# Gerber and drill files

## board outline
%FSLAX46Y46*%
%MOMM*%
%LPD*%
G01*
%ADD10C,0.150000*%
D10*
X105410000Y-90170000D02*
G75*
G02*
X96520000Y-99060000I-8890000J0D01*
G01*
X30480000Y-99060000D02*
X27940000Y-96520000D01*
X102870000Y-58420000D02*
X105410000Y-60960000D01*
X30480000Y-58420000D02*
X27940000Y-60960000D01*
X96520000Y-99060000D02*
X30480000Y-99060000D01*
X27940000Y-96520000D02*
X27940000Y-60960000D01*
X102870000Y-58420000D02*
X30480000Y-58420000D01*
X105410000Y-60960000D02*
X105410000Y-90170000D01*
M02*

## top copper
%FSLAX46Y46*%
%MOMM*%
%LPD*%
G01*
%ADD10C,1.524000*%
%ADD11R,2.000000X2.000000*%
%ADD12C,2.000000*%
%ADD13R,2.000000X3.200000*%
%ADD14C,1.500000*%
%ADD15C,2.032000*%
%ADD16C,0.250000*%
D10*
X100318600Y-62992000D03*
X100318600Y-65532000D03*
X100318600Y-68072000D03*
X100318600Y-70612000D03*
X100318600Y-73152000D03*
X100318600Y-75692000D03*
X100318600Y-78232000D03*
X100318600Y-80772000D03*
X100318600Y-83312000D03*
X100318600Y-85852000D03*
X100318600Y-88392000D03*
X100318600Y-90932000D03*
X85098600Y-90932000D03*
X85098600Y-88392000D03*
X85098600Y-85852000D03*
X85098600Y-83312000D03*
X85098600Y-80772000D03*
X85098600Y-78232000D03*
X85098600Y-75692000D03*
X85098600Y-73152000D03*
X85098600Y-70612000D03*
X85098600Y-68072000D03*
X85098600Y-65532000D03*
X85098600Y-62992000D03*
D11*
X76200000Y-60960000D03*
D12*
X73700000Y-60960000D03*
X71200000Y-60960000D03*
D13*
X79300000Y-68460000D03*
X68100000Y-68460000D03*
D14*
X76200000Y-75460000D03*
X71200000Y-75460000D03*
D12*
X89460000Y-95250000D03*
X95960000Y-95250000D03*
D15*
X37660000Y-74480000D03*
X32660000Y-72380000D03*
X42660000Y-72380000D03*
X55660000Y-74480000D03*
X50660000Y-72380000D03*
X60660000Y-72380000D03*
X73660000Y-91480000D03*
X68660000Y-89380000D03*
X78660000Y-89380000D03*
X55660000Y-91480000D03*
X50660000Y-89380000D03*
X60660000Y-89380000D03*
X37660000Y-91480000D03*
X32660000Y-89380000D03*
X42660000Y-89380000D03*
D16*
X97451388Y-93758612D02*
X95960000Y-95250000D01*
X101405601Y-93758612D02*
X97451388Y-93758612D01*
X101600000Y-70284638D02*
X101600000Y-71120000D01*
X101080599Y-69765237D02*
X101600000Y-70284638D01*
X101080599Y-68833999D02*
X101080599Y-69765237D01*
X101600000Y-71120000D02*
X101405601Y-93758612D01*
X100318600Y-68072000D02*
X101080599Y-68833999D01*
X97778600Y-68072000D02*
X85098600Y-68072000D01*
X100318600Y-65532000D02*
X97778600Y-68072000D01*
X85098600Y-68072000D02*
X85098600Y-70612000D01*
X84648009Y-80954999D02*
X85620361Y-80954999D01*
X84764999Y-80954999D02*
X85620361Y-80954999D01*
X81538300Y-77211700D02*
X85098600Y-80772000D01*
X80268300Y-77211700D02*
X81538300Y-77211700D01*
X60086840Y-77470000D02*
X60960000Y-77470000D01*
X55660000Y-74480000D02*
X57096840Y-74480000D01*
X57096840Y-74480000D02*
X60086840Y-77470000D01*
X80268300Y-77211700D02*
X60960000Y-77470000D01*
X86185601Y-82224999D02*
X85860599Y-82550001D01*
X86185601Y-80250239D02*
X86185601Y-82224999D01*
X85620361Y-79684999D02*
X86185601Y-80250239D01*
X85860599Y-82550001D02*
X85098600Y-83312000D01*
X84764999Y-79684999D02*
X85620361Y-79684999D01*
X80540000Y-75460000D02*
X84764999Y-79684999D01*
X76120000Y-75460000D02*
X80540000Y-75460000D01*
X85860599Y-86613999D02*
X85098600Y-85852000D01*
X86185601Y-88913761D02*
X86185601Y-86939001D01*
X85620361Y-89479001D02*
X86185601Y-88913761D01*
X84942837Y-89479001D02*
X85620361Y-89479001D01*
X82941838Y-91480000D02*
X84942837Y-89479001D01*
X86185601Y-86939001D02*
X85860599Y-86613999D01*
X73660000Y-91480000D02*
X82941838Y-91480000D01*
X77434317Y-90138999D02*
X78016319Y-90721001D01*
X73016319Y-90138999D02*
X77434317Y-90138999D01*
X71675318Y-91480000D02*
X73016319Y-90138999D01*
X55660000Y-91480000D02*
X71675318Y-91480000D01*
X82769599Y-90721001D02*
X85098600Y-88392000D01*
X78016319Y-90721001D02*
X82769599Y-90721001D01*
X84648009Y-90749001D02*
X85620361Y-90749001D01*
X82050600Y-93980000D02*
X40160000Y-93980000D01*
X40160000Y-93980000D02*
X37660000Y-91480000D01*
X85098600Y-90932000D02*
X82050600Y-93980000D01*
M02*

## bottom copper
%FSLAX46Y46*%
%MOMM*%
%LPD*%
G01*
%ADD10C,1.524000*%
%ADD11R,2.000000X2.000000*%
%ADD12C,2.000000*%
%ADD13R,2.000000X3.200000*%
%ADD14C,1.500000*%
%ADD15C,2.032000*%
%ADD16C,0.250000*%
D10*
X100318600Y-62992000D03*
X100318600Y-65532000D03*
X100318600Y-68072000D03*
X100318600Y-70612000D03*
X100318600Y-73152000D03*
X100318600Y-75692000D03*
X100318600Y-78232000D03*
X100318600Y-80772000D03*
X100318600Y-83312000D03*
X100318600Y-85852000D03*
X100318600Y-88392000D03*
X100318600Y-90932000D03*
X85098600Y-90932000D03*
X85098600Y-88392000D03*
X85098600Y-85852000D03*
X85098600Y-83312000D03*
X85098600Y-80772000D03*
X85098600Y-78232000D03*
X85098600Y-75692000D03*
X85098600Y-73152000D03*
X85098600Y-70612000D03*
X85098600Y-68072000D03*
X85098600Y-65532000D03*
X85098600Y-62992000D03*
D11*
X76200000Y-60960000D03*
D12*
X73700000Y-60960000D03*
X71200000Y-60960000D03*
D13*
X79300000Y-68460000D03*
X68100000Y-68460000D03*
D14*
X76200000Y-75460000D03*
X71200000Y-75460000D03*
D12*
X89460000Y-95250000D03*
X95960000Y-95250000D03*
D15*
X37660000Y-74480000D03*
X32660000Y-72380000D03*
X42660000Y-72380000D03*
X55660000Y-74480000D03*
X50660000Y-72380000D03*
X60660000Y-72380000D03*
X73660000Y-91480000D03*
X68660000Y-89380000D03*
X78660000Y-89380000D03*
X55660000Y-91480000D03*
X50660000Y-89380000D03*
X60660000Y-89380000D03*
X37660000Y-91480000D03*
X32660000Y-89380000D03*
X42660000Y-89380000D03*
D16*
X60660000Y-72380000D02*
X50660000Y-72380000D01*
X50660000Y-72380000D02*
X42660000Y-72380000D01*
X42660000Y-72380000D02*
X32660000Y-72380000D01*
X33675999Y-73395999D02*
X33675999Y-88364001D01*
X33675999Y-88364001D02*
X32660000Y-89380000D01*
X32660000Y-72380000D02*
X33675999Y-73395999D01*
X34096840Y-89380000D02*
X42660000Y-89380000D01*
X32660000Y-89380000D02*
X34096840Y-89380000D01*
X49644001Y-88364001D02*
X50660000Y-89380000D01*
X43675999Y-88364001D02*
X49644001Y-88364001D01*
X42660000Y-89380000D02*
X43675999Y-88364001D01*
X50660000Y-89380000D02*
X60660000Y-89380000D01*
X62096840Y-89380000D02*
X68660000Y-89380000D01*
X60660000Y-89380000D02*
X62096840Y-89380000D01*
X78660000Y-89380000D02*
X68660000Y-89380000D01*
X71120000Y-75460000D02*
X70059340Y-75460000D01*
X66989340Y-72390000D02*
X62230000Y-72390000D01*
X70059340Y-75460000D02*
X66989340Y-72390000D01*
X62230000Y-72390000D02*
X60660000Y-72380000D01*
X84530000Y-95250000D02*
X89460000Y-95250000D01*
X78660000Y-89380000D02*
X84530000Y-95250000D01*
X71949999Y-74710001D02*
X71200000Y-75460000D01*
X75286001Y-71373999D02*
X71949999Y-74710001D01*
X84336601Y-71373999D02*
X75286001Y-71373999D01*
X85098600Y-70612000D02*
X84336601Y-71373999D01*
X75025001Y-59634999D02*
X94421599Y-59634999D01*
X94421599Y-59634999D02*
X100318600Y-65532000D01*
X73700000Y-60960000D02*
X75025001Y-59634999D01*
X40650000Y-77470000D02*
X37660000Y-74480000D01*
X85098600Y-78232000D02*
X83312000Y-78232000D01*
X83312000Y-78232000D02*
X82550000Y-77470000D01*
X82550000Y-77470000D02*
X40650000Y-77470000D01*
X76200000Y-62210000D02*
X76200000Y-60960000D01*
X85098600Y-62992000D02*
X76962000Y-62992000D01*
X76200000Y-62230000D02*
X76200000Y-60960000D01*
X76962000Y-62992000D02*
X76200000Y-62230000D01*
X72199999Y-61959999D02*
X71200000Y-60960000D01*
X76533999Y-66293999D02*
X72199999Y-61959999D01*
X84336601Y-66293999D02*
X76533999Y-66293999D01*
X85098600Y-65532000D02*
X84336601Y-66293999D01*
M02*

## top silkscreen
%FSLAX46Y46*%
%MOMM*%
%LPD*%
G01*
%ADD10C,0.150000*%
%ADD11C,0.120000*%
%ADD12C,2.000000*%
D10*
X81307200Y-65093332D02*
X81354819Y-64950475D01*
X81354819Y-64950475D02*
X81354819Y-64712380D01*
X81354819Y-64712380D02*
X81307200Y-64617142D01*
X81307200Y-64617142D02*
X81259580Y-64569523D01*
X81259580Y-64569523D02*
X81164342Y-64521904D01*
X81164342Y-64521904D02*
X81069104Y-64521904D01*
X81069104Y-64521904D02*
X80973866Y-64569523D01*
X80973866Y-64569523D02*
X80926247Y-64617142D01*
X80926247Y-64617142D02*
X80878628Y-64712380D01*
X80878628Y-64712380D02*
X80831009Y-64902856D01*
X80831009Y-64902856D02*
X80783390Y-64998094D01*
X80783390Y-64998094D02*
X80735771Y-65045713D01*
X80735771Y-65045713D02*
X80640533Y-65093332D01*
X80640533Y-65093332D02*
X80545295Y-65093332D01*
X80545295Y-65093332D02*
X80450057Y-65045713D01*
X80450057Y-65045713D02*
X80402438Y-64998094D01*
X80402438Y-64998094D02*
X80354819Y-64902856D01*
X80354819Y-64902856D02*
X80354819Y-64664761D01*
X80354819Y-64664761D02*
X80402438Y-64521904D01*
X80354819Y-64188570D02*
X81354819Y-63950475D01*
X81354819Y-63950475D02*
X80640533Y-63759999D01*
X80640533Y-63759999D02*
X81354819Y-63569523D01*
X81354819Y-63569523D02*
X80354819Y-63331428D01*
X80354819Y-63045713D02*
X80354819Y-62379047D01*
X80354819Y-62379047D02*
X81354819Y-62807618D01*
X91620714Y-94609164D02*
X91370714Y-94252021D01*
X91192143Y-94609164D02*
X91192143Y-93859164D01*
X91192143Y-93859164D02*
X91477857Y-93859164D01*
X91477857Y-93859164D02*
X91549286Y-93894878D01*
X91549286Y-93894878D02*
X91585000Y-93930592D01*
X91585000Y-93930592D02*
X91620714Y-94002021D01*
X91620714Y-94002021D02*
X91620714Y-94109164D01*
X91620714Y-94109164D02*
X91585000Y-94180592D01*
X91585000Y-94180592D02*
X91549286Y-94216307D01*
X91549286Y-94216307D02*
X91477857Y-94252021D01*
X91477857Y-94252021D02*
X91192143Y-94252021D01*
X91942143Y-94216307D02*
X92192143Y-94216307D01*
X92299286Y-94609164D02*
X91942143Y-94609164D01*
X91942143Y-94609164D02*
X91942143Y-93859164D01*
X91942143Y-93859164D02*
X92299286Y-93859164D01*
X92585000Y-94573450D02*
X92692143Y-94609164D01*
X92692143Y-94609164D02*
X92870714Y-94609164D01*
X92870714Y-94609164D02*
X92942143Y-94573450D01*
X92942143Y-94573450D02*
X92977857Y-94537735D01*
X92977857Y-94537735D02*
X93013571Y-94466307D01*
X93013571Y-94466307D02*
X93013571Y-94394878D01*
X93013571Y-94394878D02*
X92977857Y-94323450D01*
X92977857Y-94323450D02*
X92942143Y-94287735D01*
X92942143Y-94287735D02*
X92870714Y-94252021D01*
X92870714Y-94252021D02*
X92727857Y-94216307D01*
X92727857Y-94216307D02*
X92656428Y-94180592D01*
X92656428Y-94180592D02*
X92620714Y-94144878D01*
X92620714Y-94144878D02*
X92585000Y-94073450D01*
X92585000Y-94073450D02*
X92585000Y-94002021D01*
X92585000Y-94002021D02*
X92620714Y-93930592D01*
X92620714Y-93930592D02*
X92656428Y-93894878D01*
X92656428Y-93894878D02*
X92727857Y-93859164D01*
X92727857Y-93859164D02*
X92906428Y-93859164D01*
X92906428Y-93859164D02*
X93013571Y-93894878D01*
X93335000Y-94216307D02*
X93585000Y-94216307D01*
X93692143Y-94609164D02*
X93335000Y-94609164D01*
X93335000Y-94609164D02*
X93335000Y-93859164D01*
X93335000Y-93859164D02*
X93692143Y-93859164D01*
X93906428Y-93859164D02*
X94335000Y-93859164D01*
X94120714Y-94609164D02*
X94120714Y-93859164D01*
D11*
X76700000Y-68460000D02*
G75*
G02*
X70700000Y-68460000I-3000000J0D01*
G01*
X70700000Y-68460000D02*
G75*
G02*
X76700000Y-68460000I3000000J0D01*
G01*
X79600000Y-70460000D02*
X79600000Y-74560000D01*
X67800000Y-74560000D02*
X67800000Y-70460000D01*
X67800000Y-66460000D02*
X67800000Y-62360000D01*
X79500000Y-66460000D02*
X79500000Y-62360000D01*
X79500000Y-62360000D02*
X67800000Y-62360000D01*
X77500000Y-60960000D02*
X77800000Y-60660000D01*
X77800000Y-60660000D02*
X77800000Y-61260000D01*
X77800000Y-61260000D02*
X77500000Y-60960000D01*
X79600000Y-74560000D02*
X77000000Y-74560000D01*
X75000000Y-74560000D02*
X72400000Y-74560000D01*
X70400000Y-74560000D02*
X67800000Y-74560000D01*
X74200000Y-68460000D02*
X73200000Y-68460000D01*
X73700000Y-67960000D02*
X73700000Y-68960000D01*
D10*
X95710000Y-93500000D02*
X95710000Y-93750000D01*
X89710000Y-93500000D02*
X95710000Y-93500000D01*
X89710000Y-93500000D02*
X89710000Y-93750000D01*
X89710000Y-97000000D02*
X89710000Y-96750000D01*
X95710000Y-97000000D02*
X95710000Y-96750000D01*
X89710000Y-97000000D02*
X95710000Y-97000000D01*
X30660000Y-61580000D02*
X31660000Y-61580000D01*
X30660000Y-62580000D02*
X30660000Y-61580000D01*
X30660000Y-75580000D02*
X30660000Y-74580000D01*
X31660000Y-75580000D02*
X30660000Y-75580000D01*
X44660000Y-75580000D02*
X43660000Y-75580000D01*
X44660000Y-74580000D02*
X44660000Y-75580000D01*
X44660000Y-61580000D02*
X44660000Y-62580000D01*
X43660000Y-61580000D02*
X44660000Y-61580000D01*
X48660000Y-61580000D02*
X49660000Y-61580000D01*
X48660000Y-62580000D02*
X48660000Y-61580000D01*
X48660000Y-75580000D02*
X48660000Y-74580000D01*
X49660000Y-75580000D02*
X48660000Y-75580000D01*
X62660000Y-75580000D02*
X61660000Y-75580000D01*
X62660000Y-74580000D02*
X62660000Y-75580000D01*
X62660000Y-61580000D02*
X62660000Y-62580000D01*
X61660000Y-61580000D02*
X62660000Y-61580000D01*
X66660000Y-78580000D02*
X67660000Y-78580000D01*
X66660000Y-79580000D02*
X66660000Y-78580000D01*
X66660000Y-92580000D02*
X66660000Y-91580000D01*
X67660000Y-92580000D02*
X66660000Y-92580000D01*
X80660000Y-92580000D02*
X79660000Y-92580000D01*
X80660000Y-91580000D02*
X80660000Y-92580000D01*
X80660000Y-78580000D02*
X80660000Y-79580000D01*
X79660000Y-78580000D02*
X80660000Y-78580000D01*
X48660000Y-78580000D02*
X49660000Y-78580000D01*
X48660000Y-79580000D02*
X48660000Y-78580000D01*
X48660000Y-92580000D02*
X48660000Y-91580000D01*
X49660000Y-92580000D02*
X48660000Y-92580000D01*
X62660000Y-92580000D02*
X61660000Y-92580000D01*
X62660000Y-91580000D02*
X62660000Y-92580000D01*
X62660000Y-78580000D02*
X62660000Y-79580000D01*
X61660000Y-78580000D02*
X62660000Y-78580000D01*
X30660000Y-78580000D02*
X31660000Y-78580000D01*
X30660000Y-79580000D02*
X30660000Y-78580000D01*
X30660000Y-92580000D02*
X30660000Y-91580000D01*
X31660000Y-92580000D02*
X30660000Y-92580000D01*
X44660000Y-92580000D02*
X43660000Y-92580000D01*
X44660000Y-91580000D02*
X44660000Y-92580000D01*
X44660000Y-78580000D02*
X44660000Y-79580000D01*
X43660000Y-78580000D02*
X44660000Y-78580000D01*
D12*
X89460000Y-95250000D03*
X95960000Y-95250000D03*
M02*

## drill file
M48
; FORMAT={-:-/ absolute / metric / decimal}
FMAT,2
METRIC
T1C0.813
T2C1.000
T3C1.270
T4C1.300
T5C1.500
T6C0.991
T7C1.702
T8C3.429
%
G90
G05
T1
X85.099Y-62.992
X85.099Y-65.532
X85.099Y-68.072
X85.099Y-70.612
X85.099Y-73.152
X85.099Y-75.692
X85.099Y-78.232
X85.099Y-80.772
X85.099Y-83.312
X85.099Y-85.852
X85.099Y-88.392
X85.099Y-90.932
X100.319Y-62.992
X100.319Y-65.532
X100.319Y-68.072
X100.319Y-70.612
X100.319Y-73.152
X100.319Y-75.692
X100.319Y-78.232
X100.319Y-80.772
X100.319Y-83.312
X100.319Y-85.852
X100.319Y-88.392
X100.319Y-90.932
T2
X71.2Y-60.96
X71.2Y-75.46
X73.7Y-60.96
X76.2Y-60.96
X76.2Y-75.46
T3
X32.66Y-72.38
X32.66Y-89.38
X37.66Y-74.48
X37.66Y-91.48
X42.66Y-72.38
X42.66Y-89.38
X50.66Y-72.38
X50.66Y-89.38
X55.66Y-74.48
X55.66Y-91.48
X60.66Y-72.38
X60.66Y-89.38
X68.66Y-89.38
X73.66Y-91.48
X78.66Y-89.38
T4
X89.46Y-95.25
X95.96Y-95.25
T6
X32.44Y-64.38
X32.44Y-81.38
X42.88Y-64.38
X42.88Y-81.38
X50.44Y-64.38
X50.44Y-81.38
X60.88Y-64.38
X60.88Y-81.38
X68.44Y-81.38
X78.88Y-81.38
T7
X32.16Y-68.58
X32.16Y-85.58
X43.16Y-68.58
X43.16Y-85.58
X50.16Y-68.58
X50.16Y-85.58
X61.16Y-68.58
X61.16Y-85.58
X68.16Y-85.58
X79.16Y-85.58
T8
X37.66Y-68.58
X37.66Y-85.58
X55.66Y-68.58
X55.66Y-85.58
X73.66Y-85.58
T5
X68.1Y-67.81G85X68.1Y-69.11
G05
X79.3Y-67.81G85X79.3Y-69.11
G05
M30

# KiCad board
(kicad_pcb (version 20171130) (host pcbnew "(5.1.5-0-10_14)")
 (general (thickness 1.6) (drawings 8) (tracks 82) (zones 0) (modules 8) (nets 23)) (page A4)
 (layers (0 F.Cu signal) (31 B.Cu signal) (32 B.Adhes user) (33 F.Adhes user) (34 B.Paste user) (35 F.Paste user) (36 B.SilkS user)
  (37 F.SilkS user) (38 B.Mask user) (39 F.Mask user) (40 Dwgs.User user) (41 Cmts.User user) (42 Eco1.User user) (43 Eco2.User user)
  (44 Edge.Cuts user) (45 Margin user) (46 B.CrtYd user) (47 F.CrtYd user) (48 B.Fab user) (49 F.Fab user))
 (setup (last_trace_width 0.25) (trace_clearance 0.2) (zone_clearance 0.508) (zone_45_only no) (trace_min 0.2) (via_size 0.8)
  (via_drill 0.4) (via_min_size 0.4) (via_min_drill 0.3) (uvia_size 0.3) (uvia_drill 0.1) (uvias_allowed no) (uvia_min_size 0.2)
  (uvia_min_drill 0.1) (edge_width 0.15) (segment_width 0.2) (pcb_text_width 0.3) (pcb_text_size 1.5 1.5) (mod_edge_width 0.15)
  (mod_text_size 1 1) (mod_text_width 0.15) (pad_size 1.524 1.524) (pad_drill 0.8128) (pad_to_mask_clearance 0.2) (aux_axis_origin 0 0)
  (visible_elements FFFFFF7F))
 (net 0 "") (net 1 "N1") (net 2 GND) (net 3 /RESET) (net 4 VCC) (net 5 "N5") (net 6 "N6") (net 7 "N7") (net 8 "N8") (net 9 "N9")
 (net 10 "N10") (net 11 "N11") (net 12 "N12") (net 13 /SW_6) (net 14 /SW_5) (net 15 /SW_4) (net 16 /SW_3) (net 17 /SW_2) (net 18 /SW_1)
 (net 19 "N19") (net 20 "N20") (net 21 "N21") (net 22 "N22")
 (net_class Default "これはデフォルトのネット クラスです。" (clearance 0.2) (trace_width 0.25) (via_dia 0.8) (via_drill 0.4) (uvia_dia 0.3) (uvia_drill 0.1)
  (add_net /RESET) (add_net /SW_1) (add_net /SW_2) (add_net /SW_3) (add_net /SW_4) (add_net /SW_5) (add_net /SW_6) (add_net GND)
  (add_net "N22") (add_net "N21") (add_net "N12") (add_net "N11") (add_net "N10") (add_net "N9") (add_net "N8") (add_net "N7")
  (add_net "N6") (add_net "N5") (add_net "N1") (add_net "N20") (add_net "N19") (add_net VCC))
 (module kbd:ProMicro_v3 (layer B.Cu) (at 92.71 77.47 180)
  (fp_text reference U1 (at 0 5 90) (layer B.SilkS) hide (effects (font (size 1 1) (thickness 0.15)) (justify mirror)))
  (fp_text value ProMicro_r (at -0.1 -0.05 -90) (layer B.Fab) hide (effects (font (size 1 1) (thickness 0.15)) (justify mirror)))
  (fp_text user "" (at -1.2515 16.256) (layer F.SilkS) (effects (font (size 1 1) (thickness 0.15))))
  (pad 24 thru_hole circle (at -7.6086 14.478 180) (size 1.524 1.524) (drill 0.8128) (layers *.Cu *.Mask B.SilkS) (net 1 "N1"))
  (pad 23 thru_hole circle (at -7.6086 11.938 180) (size 1.524 1.524) (drill 0.8128) (layers *.Cu *.Mask B.SilkS) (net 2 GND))
  (pad 22 thru_hole circle (at -7.6086 9.398 180) (size 1.524 1.524) (drill 0.8128) (layers *.Cu *.Mask B.SilkS) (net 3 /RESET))
  (pad 21 thru_hole circle (at -7.6086 6.858 180) (size 1.524 1.524) (drill 0.8128) (layers *.Cu *.Mask B.SilkS) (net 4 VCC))
  (pad 20 thru_hole circle (at -7.6086 4.318 180) (size 1.524 1.524) (drill 0.8128) (layers *.Cu *.Mask B.SilkS) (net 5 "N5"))
  (pad 19 thru_hole circle (at -7.6086 1.778 180) (size 1.524 1.524) (drill 0.8128) (layers *.Cu *.Mask B.SilkS) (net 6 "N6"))
  (pad 18 thru_hole circle (at -7.6086 -0.762 180) (size 1.524 1.524) (drill 0.8128) (layers *.Cu *.Mask B.SilkS) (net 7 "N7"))
  (pad 17 thru_hole circle (at -7.6086 -3.302 180) (size 1.524 1.524) (drill 0.8128) (layers *.Cu *.Mask B.SilkS) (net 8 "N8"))
  (pad 16 thru_hole circle (at -7.6086 -5.842 180) (size 1.524 1.524) (drill 0.8128) (layers *.Cu *.Mask B.SilkS) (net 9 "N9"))
  (pad 15 thru_hole circle (at -7.6086 -8.382 180) (size 1.524 1.524) (drill 0.8128) (layers *.Cu *.Mask B.SilkS) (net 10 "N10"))
  (pad 14 thru_hole circle (at -7.6086 -10.922 180) (size 1.524 1.524) (drill 0.8128) (layers *.Cu *.Mask B.SilkS) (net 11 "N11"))
  (pad 13 thru_hole circle (at -7.6086 -13.462 180) (size 1.524 1.524) (drill 0.8128) (layers *.Cu *.Mask B.SilkS) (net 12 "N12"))
  (pad 12 thru_hole circle (at 7.6114 -13.462 180) (size 1.524 1.524) (drill 0.8128) (layers *.Cu *.Mask B.SilkS) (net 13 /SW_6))
  (pad 11 thru_hole circle (at 7.6114 -10.922 180) (size 1.524 1.524) (drill 0.8128) (layers *.Cu *.Mask B.SilkS) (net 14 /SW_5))
  (pad 10 thru_hole circle (at 7.6114 -8.382 180) (size 1.524 1.524) (drill 0.8128) (layers *.Cu *.Mask B.SilkS) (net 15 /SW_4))
  (pad 9 thru_hole circle (at 7.6114 -5.842 180) (size 1.524 1.524) (drill 0.8128) (layers *.Cu *.Mask B.SilkS) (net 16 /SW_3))
  (pad 8 thru_hole circle (at 7.6114 -3.302 180) (size 1.524 1.524) (drill 0.8128) (layers *.Cu *.Mask B.SilkS) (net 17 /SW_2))
  (pad 7 thru_hole circle (at 7.6114 -0.762 180) (size 1.524 1.524) (drill 0.8128) (layers *.Cu *.Mask B.SilkS) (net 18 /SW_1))
  (pad 6 thru_hole circle (at 7.6114 1.778 180) (size 1.524 1.524) (drill 0.8128) (layers *.Cu *.Mask B.SilkS) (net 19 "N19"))
  (pad 5 thru_hole circle (at 7.6114 4.318 180) (size 1.524 1.524) (drill 0.8128) (layers *.Cu *.Mask B.SilkS) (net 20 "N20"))
  (pad 4 thru_hole circle (at 7.6114 6.858 180) (size 1.524 1.524) (drill 0.8128) (layers *.Cu *.Mask B.SilkS) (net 2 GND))
  (pad 3 thru_hole circle (at 7.6114 9.398 180) (size 1.524 1.524) (drill 0.8128) (layers *.Cu *.Mask B.SilkS) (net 2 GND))
  (pad 2 thru_hole circle (at 7.6114 11.938 180) (size 1.524 1.524) (drill 0.8128) (layers *.Cu *.Mask B.SilkS) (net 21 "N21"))
  (pad 1 thru_hole circle (at 7.6114 14.478 180) (size 1.524 1.524) (drill 0.8128) (layers *.Cu *.Mask B.SilkS) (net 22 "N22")))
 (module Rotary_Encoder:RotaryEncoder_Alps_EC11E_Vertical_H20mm (layer F.Cu) (at 76.2 60.96 270)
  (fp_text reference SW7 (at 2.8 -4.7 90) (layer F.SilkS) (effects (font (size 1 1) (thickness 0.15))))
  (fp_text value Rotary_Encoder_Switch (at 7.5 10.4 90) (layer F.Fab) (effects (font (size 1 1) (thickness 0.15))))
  (fp_circle (center 7.5 2.5) (end 10.5 2.5) (layer F.SilkS) (width 0.12))
  (fp_line (start 9.5 -3.4) (end 13.6 -3.4) (layer F.SilkS) (width 0.12))
  (fp_line (start 13.6 8.4) (end 9.5 8.4) (layer F.SilkS) (width 0.12))
  (fp_line (start 5.5 8.4) (end 1.4 8.4) (layer F.SilkS) (width 0.12))
  (fp_line (start 5.5 -3.3) (end 1.4 -3.3) (layer F.SilkS) (width 0.12))
  (fp_line (start 1.4 -3.3) (end 1.4 8.4) (layer F.SilkS) (width 0.12))
  (fp_line (start 0 -1.3) (end -0.3 -1.6) (layer F.SilkS) (width 0.12))
  (fp_line (start -0.3 -1.6) (end 0.3 -1.6) (layer F.SilkS) (width 0.12))
  (fp_line (start 0.3 -1.6) (end 0 -1.3) (layer F.SilkS) (width 0.12))
  (fp_line (start 13.6 -3.4) (end 13.6 -0.8) (layer F.SilkS) (width 0.12))
  (fp_line (start 13.6 1.2) (end 13.6 3.8) (layer F.SilkS) (width 0.12))
  (fp_line (start 13.6 5.8) (end 13.6 8.4) (layer F.SilkS) (width 0.12))
  (fp_line (start 7.5 2) (end 7.5 3) (layer F.SilkS) (width 0.12))
  (fp_line (start 7 2.5) (end 8 2.5) (layer F.SilkS) (width 0.12))
  (pad A thru_hole rect (at 0 0 270) (size 2 2) (drill 1) (layers *.Cu *.Mask) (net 22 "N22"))
  (pad C thru_hole circle (at 0 2.5 270) (size 2 2) (drill 1) (layers *.Cu *.Mask) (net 2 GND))
  (pad B thru_hole circle (at 0 5 270) (size 2 2) (drill 1) (layers *.Cu *.Mask) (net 21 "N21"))
  (pad MP thru_hole rect (at 7.5 -3.1 270) (size 3.2 2) (drill oval 2.8 1.5) (layers *.Cu *.Mask))
  (pad MP thru_hole rect (at 7.5 8.1 270) (size 3.2 2) (drill oval 2.8 1.5) (layers *.Cu *.Mask))
  (pad "" thru_hole circle (at 14.5 0 270) (size 1.5 1.5) (drill 1) (layers *.Cu *.Mask) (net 16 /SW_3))
  (pad "" thru_hole circle (at 14.5 5 270) (size 1.5 1.5) (drill 1) (layers *.Cu *.Mask) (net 2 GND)))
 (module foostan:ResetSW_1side (layer F.Cu) (at 92.71 95.25)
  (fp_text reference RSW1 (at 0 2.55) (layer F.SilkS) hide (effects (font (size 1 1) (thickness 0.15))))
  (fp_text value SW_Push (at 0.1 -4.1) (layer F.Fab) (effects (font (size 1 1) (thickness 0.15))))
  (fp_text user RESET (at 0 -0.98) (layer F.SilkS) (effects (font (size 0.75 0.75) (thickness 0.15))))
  (fp_line (start 3 -1.75) (end 3 -1.5) (layer F.SilkS) (width 0.15))
  (fp_line (start -3 -1.75) (end 3 -1.75) (layer F.SilkS) (width 0.15))
  (fp_line (start -3 -1.75) (end -3 -1.5) (layer F.SilkS) (width 0.15))
  (fp_line (start -3 1.75) (end -3 1.5) (layer F.SilkS) (width 0.15))
  (fp_line (start 3 1.75) (end 3 1.5) (layer F.SilkS) (width 0.15))
  (fp_line (start -3 1.75) (end 3 1.75) (layer F.SilkS) (width 0.15))
  (pad 2 thru_hole circle (at -3.25 0) (size 2 2) (drill 1.3) (layers *.Cu F.SilkS B.Mask) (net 2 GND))
  (pad 1 thru_hole circle (at 3.25 0) (size 2 2) (drill 1.3) (layers *.Cu F.SilkS B.Mask) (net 3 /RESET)))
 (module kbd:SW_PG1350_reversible (layer F.Cu) (at 37.66 68.58)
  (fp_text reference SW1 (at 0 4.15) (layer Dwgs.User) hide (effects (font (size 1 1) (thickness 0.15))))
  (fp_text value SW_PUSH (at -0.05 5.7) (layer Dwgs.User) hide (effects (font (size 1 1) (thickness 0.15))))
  (fp_line (start -7 -7) (end -6 -7) (layer F.SilkS) (width 0.15))
  (fp_line (start -7 -6) (end -7 -7) (layer F.SilkS) (width 0.15))
  (fp_line (start -7 7) (end -7 6) (layer F.SilkS) (width 0.15))
  (fp_line (start -6 7) (end -7 7) (layer F.SilkS) (width 0.15)) (fp_line (start 7 7) (end 6 7) (layer F.SilkS) (width 0.15))
  (fp_line (start 7 6) (end 7 7) (layer F.SilkS) (width 0.15))
  (fp_line (start 7 -7) (end 7 -6) (layer F.SilkS) (width 0.15))
  (fp_line (start 6 -7) (end 7 -7) (layer F.SilkS) (width 0.15))
  (pad "" np_thru_hole circle (at -5.5 0) (size 1.7018 1.7018) (drill 1.7018) (layers *.Cu *.Mask))
  (pad "" np_thru_hole circle (at 5.5 0) (size 1.7018 1.7018) (drill 1.7018) (layers *.Cu *.Mask))
  (pad "" np_thru_hole circle (at 5.22 -4.2) (size 0.9906 0.9906) (drill 0.9906) (layers *.Cu *.Mask))
  (pad 1 thru_hole circle (at 0 5.9) (size 2.032 2.032) (drill 1.27) (layers *.Cu *.Mask) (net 18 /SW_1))
  (pad 2 thru_hole circle (at -5 3.8) (size 2.032 2.032) (drill 1.27) (layers *.Cu *.Mask) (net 2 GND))
  (pad "" np_thru_hole circle (at 0 0) (size 3.429 3.429) (drill 3.429) (layers *.Cu *.Mask))
  (pad 2 thru_hole circle (at 5 3.8) (size 2.032 2.032) (drill 1.27) (layers *.Cu *.Mask) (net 2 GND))
  (pad "" np_thru_hole circle (at -5.22 -4.2) (size 0.9906 0.9906) (drill 0.9906) (layers *.Cu *.Mask)))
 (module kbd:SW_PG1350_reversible (layer F.Cu) (at 55.66 68.58)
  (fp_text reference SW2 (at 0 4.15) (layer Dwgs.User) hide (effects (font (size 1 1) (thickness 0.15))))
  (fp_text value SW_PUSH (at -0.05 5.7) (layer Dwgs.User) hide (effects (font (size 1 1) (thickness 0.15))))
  (fp_line (start -7 -7) (end -6 -7) (layer F.SilkS) (width 0.15))
  (fp_line (start -7 -6) (end -7 -7) (layer F.SilkS) (width 0.15))
  (fp_line (start -7 7) (end -7 6) (layer F.SilkS) (width 0.15))
  (fp_line (start -6 7) (end -7 7) (layer F.SilkS) (width 0.15)) (fp_line (start 7 7) (end 6 7) (layer F.SilkS) (width 0.15))
  (fp_line (start 7 6) (end 7 7) (layer F.SilkS) (width 0.15))
  (fp_line (start 7 -7) (end 7 -6) (layer F.SilkS) (width 0.15))
  (fp_line (start 6 -7) (end 7 -7) (layer F.SilkS) (width 0.15))
  (pad "" np_thru_hole circle (at -5.5 0) (size 1.7018 1.7018) (drill 1.7018) (layers *.Cu *.Mask))
  (pad "" np_thru_hole circle (at 5.5 0) (size 1.7018 1.7018) (drill 1.7018) (layers *.Cu *.Mask))
  (pad "" np_thru_hole circle (at 5.22 -4.2) (size 0.9906 0.9906) (drill 0.9906) (layers *.Cu *.Mask))
  (pad 1 thru_hole circle (at 0 5.9) (size 2.032 2.032) (drill 1.27) (layers *.Cu *.Mask) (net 17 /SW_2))
  (pad 2 thru_hole circle (at -5 3.8) (size 2.032 2.032) (drill 1.27) (layers *.Cu *.Mask) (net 2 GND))
  (pad "" np_thru_hole circle (at 0 0) (size 3.429 3.429) (drill 3.429) (layers *.Cu *.Mask))
  (pad 2 thru_hole circle (at 5 3.8) (size 2.032 2.032) (drill 1.27) (layers *.Cu *.Mask) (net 2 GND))
  (pad "" np_thru_hole circle (at -5.22 -4.2) (size 0.9906 0.9906) (drill 0.9906) (layers *.Cu *.Mask)))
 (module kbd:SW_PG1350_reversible (layer F.Cu) (at 73.66 85.58)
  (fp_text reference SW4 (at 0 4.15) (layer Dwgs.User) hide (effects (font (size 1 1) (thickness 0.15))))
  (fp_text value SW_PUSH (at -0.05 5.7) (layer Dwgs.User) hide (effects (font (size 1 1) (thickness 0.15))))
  (fp_line (start -7 -7) (end -6 -7) (layer F.SilkS) (width 0.15))
  (fp_line (start -7 -6) (end -7 -7) (layer F.SilkS) (width 0.15))
  (fp_line (start -7 7) (end -7 6) (layer F.SilkS) (width 0.15))
  (fp_line (start -6 7) (end -7 7) (layer F.SilkS) (width 0.15)) (fp_line (start 7 7) (end 6 7) (layer F.SilkS) (width 0.15))
  (fp_line (start 7 6) (end 7 7) (layer F.SilkS) (width 0.15))
  (fp_line (start 7 -7) (end 7 -6) (layer F.SilkS) (width 0.15))
  (fp_line (start 6 -7) (end 7 -7) (layer F.SilkS) (width 0.15))
  (pad "" np_thru_hole circle (at -5.5 0) (size 1.7018 1.7018) (drill 1.7018) (layers *.Cu *.Mask))
  (pad "" np_thru_hole circle (at 5.5 0) (size 1.7018 1.7018) (drill 1.7018) (layers *.Cu *.Mask))
  (pad "" np_thru_hole circle (at 5.22 -4.2) (size 0.9906 0.9906) (drill 0.9906) (layers *.Cu *.Mask))
  (pad 1 thru_hole circle (at 0 5.9) (size 2.032 2.032) (drill 1.27) (layers *.Cu *.Mask) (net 15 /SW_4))
  (pad 2 thru_hole circle (at -5 3.8) (size 2.032 2.032) (drill 1.27) (layers *.Cu *.Mask) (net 2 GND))
  (pad "" np_thru_hole circle (at 0 0) (size 3.429 3.429) (drill 3.429) (layers *.Cu *.Mask))
  (pad 2 thru_hole circle (at 5 3.8) (size 2.032 2.032) (drill 1.27) (layers *.Cu *.Mask) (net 2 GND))
  (pad "" np_thru_hole circle (at -5.22 -4.2) (size 0.9906 0.9906) (drill 0.9906) (layers *.Cu *.Mask)))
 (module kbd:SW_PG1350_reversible (layer F.Cu) (at 55.66 85.58)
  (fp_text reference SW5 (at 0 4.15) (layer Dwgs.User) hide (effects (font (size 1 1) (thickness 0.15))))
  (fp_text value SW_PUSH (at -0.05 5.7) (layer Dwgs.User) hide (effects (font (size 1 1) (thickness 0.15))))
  (fp_line (start -7 -7) (end -6 -7) (layer F.SilkS) (width 0.15))
  (fp_line (start -7 -6) (end -7 -7) (layer F.SilkS) (width 0.15))
  (fp_line (start -7 7) (end -7 6) (layer F.SilkS) (width 0.15))
  (fp_line (start -6 7) (end -7 7) (layer F.SilkS) (width 0.15)) (fp_line (start 7 7) (end 6 7) (layer F.SilkS) (width 0.15))
  (fp_line (start 7 6) (end 7 7) (layer F.SilkS) (width 0.15))
  (fp_line (start 7 -7) (end 7 -6) (layer F.SilkS) (width 0.15))
  (fp_line (start 6 -7) (end 7 -7) (layer F.SilkS) (width 0.15))
  (pad "" np_thru_hole circle (at -5.5 0) (size 1.7018 1.7018) (drill 1.7018) (layers *.Cu *.Mask))
  (pad "" np_thru_hole circle (at 5.5 0) (size 1.7018 1.7018) (drill 1.7018) (layers *.Cu *.Mask))
  (pad "" np_thru_hole circle (at 5.22 -4.2) (size 0.9906 0.9906) (drill 0.9906) (layers *.Cu *.Mask))
  (pad 1 thru_hole circle (at 0 5.9) (size 2.032 2.032) (drill 1.27) (layers *.Cu *.Mask) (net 14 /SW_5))
  (pad 2 thru_hole circle (at -5 3.8) (size 2.032 2.032) (drill 1.27) (layers *.Cu *.Mask) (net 2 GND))
  (pad "" np_thru_hole circle (at 0 0) (size 3.429 3.429) (drill 3.429) (layers *.Cu *.Mask))
  (pad 2 thru_hole circle (at 5 3.8) (size 2.032 2.032) (drill 1.27) (layers *.Cu *.Mask) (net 2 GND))
  (pad "" np_thru_hole circle (at -5.22 -4.2) (size 0.9906 0.9906) (drill 0.9906) (layers *.Cu *.Mask)))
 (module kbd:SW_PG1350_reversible (layer F.Cu) (at 37.66 85.58)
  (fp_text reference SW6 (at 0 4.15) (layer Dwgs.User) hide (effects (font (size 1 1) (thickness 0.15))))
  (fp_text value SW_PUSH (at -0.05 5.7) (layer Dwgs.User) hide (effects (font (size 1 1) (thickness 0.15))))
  (fp_line (start -7 -7) (end -6 -7) (layer F.SilkS) (width 0.15))
  (fp_line (start -7 -6) (end -7 -7) (layer F.SilkS) (width 0.15))
  (fp_line (start -7 7) (end -7 6) (layer F.SilkS) (width 0.15))
  (fp_line (start -6 7) (end -7 7) (layer F.SilkS) (width 0.15)) (fp_line (start 7 7) (end 6 7) (layer F.SilkS) (width 0.15))
  (fp_line (start 7 6) (end 7 7) (layer F.SilkS) (width 0.15))
  (fp_line (start 7 -7) (end 7 -6) (layer F.SilkS) (width 0.15))
  (fp_line (start 6 -7) (end 7 -7) (layer F.SilkS) (width 0.15))
  (pad "" np_thru_hole circle (at -5.5 0) (size 1.7018 1.7018) (drill 1.7018) (layers *.Cu *.Mask))
  (pad "" np_thru_hole circle (at 5.5 0) (size 1.7018 1.7018) (drill 1.7018) (layers *.Cu *.Mask))
  (pad "" np_thru_hole circle (at 5.22 -4.2) (size 0.9906 0.9906) (drill 0.9906) (layers *.Cu *.Mask))
  (pad 1 thru_hole circle (at 0 5.9) (size 2.032 2.032) (drill 1.27) (layers *.Cu *.Mask) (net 13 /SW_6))
  (pad 2 thru_hole circle (at -5 3.8) (size 2.032 2.032) (drill 1.27) (layers *.Cu *.Mask) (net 2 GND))
  (pad "" np_thru_hole circle (at 0 0) (size 3.429 3.429) (drill 3.429) (layers *.Cu *.Mask))
  (pad 2 thru_hole circle (at 5 3.8) (size 2.032 2.032) (drill 1.27) (layers *.Cu *.Mask) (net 2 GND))
  (pad "" np_thru_hole circle (at -5.22 -4.2) (size 0.9906 0.9906) (drill 0.9906) (layers *.Cu *.Mask)))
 (gr_arc (start 96.52 90.17) (end 96.52 99.06) (angle -90) (layer Edge.Cuts) (width 0.15))
 (gr_line (start 30.48 99.06) (end 27.94 96.52) (layer Edge.Cuts) (width 0.15))
 (gr_line (start 102.87 58.42) (end 105.41 60.96) (layer Edge.Cuts) (width 0.15))
 (gr_line (start 30.48 58.42) (end 27.94 60.96) (layer Edge.Cuts) (width 0.15))
 (gr_line (start 96.52 99.06) (end 30.48 99.06) (layer Edge.Cuts) (width 0.15))
 (gr_line (start 27.94 96.52) (end 27.94 60.96) (layer Edge.Cuts) (width 0.15))
 (gr_line (start 102.87 58.42) (end 30.48 58.42) (layer Edge.Cuts) (width 0.15))
 (gr_line (start 105.41 60.96) (end 105.41 90.17) (layer Edge.Cuts) (width 0.15))
 (segment (start 97.451388 93.758612) (end 95.96 95.25) (width 0.25) (layer F.Cu) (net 3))
 (segment (start 101.405601 93.758612) (end 97.451388 93.758612) (width 0.25) (layer F.Cu) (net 3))
 (segment (start 101.6 70.284638) (end 101.6 71.12) (width 0.25) (layer F.Cu) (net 3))
 (segment (start 101.080599 69.765237) (end 101.6 70.284638) (width 0.25) (layer F.Cu) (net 3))
 (segment (start 101.080599 68.833999) (end 101.080599 69.765237) (width 0.25) (layer F.Cu) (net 3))
 (segment (start 101.6 71.12) (end 101.405601 93.758612) (width 0.25) (layer F.Cu) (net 3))
 (segment (start 100.3186 68.072) (end 101.080599 68.833999) (width 0.25) (layer F.Cu) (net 3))
 (segment (start 60.66 72.38) (end 50.66 72.38) (width 0.25) (layer B.Cu) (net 2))
 (segment (start 50.66 72.38) (end 42.66 72.38) (width 0.25) (layer B.Cu) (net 2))
 (segment (start 42.66 72.38) (end 32.66 72.38) (width 0.25) (layer B.Cu) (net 2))
 (segment (start 33.675999 73.395999) (end 33.675999 88.364001) (width 0.25) (layer B.Cu) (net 2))
 (segment (start 33.675999 88.364001) (end 32.66 89.38) (width 0.25) (layer B.Cu) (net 2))
 (segment (start 32.66 72.38) (end 33.675999 73.395999) (width 0.25) (layer B.Cu) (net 2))
 (segment (start 34.09684 89.38) (end 42.66 89.38) (width 0.25) (layer B.Cu) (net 2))
 (segment (start 32.66 89.38) (end 34.09684 89.38) (width 0.25) (layer B.Cu) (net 2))
 (segment (start 49.644001 88.364001) (end 50.66 89.38) (width 0.25) (layer B.Cu) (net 2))
 (segment (start 43.675999 88.364001) (end 49.644001 88.364001) (width 0.25) (layer B.Cu) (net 2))
 (segment (start 42.66 89.38) (end 43.675999 88.364001) (width 0.25) (layer B.Cu) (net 2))
 (segment (start 50.66 89.38) (end 60.66 89.38) (width 0.25) (layer B.Cu) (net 2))
 (segment (start 62.09684 89.38) (end 68.66 89.38) (width 0.25) (layer B.Cu) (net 2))
 (segment (start 60.66 89.38) (end 62.09684 89.38) (width 0.25) (layer B.Cu) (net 2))
 (segment (start 78.66 89.38) (end 68.66 89.38) (width 0.25) (layer B.Cu) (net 2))
 (segment (start 71.12 75.46) (end 70.05934 75.46) (width 0.25) (layer B.Cu) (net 2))
 (segment (start 66.98934 72.39) (end 62.23 72.39) (width 0.25) (layer B.Cu) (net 2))
 (segment (start 70.05934 75.46) (end 66.98934 72.39) (width 0.25) (layer B.Cu) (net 2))
 (segment (start 62.23 72.39) (end 60.66 72.38) (width 0.25) (layer B.Cu) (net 2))
 (segment (start 84.53 95.25) (end 89.46 95.25) (width 0.25) (layer B.Cu) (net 2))
 (segment (start 78.66 89.38) (end 84.53 95.25) (width 0.25) (layer B.Cu) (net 2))
 (segment (start 71.949999 74.710001) (end 71.2 75.46) (width 0.25) (layer B.Cu) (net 2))
 (segment (start 75.286001 71.373999) (end 71.949999 74.710001) (width 0.25) (layer B.Cu) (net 2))
 (segment (start 84.336601 71.373999) (end 75.286001 71.373999) (width 0.25) (layer B.Cu) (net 2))
 (segment (start 85.0986 70.612) (end 84.336601 71.373999) (width 0.25) (layer B.Cu) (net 2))
 (segment (start 97.7786 68.072) (end 85.0986 68.072) (width 0.25) (layer F.Cu) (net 2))
 (segment (start 100.3186 65.532) (end 97.7786 68.072) (width 0.25) (layer F.Cu) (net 2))
 (segment (start 85.0986 68.072) (end 85.0986 70.612) (width 0.25) (layer F.Cu) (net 2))
 (segment (start 75.025001 59.634999) (end 94.421599 59.634999) (width 0.25) (layer B.Cu) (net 2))
 (segment (start 94.421599 59.634999) (end 100.3186 65.532) (width 0.25) (layer B.Cu) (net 2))
 (segment (start 73.7 60.96) (end 75.025001 59.634999) (width 0.25) (layer B.Cu) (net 2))
 (segment (start 40.65 77.47) (end 37.66 74.48) (width 0.25) (layer B.Cu) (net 18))
 (segment (start 85.0986 78.232) (end 83.312 78.232) (width 0.25) (layer B.Cu) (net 18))
 (segment (start 83.312 78.232) (end 82.55 77.47) (width 0.25) (layer B.Cu) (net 18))
 (segment (start 82.55 77.47) (end 40.65 77.47) (width 0.25) (layer B.Cu) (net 18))
 (segment (start 84.648009 80.954999) (end 85.620361 80.954999) (width 0.25) (layer F.Cu) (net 17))
 (segment (start 84.764999 80.954999) (end 85.620361 80.954999) (width 0.25) (layer F.Cu) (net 17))
 (segment (start 81.5383 77.2117) (end 85.0986 80.772) (width 0.25) (layer F.Cu) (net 17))
 (segment (start 80.2683 77.2117) (end 81.5383 77.2117) (width 0.25) (layer F.Cu) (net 17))
 (segment (start 60.08684 77.47) (end 60.96 77.47) (width 0.25) (layer F.Cu) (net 17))
 (segment (start 55.66 74.48) (end 57.09684 74.48) (width 0.25) (layer F.Cu) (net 17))
 (segment (start 57.09684 74.48) (end 60.08684 77.47) (width 0.25) (layer F.Cu) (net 17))
 (segment (start 80.2683 77.2117) (end 60.96 77.47) (width 0.25) (layer F.Cu) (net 17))
 (segment (start 86.185601 82.224999) (end 85.860599 82.550001) (width 0.25) (layer F.Cu) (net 16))
 (segment (start 86.185601 80.250239) (end 86.185601 82.224999) (width 0.25) (layer F.Cu) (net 16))
 (segment (start 85.620361 79.684999) (end 86.185601 80.250239) (width 0.25) (layer F.Cu) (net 16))
 (segment (start 85.860599 82.550001) (end 85.0986 83.312) (width 0.25) (layer F.Cu) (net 16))
 (segment (start 84.764999 79.684999) (end 85.620361 79.684999) (width 0.25) (layer F.Cu) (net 16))
 (segment (start 80.54 75.46) (end 84.764999 79.684999) (width 0.25) (layer F.Cu) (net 16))
 (segment (start 76.12 75.46) (end 80.54 75.46) (width 0.25) (layer F.Cu) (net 16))
 (segment (start 85.860599 86.613999) (end 85.0986 85.852) (width 0.25) (layer F.Cu) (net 15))
 (segment (start 86.185601 88.913761) (end 86.185601 86.939001) (width 0.25) (layer F.Cu) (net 15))
 (segment (start 85.620361 89.479001) (end 86.185601 88.913761) (width 0.25) (layer F.Cu) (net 15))
 (segment (start 84.942837 89.479001) (end 85.620361 89.479001) (width 0.25) (layer F.Cu) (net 15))
 (segment (start 82.941838 91.48) (end 84.942837 89.479001) (width 0.25) (layer F.Cu) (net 15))
 (segment (start 86.185601 86.939001) (end 85.860599 86.613999) (width 0.25) (layer F.Cu) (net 15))
 (segment (start 73.66 91.48) (end 82.941838 91.48) (width 0.25) (layer F.Cu) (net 15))
 (segment (start 77.434317 90.138999) (end 78.016319 90.721001) (width 0.25) (layer F.Cu) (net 14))
 (segment (start 73.016319 90.138999) (end 77.434317 90.138999) (width 0.25) (layer F.Cu) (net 14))
 (segment (start 71.675318 91.48) (end 73.016319 90.138999) (width 0.25) (layer F.Cu) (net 14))
 (segment (start 55.66 91.48) (end 71.675318 91.48) (width 0.25) (layer F.Cu) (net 14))
 (segment (start 82.769599 90.721001) (end 85.0986 88.392) (width 0.25) (layer F.Cu) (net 14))
 (segment (start 78.016319 90.721001) (end 82.769599 90.721001) (width 0.25) (layer F.Cu) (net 14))
 (segment (start 84.648009 90.749001) (end 85.620361 90.749001) (width 0.25) (layer F.Cu) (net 13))
 (segment (start 82.0506 93.98) (end 40.16 93.98) (width 0.25) (layer F.Cu) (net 13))
 (segment (start 40.16 93.98) (end 37.66 91.48) (width 0.25) (layer F.Cu) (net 13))
 (segment (start 85.0986 90.932) (end 82.0506 93.98) (width 0.25) (layer F.Cu) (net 13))
 (segment (start 76.2 62.21) (end 76.2 60.96) (width 0.25) (layer B.Cu) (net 22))
 (segment (start 85.0986 62.992) (end 76.962 62.992) (width 0.25) (layer B.Cu) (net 22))
 (segment (start 76.2 62.23) (end 76.2 60.96) (width 0.25) (layer B.Cu) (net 22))
 (segment (start 76.962 62.992) (end 76.2 62.23) (width 0.25) (layer B.Cu) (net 22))
 (segment (start 72.199999 61.959999) (end 71.2 60.96) (width 0.25) (layer B.Cu) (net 21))
 (segment (start 76.533999 66.293999) (end 72.199999 61.959999) (width 0.25) (layer B.Cu) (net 21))
 (segment (start 84.336601 66.293999) (end 76.533999 66.293999) (width 0.25) (layer B.Cu) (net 21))
 (segment (start 85.0986 65.532) (end 84.336601 66.293999) (width 0.25) (layer B.Cu) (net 21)))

